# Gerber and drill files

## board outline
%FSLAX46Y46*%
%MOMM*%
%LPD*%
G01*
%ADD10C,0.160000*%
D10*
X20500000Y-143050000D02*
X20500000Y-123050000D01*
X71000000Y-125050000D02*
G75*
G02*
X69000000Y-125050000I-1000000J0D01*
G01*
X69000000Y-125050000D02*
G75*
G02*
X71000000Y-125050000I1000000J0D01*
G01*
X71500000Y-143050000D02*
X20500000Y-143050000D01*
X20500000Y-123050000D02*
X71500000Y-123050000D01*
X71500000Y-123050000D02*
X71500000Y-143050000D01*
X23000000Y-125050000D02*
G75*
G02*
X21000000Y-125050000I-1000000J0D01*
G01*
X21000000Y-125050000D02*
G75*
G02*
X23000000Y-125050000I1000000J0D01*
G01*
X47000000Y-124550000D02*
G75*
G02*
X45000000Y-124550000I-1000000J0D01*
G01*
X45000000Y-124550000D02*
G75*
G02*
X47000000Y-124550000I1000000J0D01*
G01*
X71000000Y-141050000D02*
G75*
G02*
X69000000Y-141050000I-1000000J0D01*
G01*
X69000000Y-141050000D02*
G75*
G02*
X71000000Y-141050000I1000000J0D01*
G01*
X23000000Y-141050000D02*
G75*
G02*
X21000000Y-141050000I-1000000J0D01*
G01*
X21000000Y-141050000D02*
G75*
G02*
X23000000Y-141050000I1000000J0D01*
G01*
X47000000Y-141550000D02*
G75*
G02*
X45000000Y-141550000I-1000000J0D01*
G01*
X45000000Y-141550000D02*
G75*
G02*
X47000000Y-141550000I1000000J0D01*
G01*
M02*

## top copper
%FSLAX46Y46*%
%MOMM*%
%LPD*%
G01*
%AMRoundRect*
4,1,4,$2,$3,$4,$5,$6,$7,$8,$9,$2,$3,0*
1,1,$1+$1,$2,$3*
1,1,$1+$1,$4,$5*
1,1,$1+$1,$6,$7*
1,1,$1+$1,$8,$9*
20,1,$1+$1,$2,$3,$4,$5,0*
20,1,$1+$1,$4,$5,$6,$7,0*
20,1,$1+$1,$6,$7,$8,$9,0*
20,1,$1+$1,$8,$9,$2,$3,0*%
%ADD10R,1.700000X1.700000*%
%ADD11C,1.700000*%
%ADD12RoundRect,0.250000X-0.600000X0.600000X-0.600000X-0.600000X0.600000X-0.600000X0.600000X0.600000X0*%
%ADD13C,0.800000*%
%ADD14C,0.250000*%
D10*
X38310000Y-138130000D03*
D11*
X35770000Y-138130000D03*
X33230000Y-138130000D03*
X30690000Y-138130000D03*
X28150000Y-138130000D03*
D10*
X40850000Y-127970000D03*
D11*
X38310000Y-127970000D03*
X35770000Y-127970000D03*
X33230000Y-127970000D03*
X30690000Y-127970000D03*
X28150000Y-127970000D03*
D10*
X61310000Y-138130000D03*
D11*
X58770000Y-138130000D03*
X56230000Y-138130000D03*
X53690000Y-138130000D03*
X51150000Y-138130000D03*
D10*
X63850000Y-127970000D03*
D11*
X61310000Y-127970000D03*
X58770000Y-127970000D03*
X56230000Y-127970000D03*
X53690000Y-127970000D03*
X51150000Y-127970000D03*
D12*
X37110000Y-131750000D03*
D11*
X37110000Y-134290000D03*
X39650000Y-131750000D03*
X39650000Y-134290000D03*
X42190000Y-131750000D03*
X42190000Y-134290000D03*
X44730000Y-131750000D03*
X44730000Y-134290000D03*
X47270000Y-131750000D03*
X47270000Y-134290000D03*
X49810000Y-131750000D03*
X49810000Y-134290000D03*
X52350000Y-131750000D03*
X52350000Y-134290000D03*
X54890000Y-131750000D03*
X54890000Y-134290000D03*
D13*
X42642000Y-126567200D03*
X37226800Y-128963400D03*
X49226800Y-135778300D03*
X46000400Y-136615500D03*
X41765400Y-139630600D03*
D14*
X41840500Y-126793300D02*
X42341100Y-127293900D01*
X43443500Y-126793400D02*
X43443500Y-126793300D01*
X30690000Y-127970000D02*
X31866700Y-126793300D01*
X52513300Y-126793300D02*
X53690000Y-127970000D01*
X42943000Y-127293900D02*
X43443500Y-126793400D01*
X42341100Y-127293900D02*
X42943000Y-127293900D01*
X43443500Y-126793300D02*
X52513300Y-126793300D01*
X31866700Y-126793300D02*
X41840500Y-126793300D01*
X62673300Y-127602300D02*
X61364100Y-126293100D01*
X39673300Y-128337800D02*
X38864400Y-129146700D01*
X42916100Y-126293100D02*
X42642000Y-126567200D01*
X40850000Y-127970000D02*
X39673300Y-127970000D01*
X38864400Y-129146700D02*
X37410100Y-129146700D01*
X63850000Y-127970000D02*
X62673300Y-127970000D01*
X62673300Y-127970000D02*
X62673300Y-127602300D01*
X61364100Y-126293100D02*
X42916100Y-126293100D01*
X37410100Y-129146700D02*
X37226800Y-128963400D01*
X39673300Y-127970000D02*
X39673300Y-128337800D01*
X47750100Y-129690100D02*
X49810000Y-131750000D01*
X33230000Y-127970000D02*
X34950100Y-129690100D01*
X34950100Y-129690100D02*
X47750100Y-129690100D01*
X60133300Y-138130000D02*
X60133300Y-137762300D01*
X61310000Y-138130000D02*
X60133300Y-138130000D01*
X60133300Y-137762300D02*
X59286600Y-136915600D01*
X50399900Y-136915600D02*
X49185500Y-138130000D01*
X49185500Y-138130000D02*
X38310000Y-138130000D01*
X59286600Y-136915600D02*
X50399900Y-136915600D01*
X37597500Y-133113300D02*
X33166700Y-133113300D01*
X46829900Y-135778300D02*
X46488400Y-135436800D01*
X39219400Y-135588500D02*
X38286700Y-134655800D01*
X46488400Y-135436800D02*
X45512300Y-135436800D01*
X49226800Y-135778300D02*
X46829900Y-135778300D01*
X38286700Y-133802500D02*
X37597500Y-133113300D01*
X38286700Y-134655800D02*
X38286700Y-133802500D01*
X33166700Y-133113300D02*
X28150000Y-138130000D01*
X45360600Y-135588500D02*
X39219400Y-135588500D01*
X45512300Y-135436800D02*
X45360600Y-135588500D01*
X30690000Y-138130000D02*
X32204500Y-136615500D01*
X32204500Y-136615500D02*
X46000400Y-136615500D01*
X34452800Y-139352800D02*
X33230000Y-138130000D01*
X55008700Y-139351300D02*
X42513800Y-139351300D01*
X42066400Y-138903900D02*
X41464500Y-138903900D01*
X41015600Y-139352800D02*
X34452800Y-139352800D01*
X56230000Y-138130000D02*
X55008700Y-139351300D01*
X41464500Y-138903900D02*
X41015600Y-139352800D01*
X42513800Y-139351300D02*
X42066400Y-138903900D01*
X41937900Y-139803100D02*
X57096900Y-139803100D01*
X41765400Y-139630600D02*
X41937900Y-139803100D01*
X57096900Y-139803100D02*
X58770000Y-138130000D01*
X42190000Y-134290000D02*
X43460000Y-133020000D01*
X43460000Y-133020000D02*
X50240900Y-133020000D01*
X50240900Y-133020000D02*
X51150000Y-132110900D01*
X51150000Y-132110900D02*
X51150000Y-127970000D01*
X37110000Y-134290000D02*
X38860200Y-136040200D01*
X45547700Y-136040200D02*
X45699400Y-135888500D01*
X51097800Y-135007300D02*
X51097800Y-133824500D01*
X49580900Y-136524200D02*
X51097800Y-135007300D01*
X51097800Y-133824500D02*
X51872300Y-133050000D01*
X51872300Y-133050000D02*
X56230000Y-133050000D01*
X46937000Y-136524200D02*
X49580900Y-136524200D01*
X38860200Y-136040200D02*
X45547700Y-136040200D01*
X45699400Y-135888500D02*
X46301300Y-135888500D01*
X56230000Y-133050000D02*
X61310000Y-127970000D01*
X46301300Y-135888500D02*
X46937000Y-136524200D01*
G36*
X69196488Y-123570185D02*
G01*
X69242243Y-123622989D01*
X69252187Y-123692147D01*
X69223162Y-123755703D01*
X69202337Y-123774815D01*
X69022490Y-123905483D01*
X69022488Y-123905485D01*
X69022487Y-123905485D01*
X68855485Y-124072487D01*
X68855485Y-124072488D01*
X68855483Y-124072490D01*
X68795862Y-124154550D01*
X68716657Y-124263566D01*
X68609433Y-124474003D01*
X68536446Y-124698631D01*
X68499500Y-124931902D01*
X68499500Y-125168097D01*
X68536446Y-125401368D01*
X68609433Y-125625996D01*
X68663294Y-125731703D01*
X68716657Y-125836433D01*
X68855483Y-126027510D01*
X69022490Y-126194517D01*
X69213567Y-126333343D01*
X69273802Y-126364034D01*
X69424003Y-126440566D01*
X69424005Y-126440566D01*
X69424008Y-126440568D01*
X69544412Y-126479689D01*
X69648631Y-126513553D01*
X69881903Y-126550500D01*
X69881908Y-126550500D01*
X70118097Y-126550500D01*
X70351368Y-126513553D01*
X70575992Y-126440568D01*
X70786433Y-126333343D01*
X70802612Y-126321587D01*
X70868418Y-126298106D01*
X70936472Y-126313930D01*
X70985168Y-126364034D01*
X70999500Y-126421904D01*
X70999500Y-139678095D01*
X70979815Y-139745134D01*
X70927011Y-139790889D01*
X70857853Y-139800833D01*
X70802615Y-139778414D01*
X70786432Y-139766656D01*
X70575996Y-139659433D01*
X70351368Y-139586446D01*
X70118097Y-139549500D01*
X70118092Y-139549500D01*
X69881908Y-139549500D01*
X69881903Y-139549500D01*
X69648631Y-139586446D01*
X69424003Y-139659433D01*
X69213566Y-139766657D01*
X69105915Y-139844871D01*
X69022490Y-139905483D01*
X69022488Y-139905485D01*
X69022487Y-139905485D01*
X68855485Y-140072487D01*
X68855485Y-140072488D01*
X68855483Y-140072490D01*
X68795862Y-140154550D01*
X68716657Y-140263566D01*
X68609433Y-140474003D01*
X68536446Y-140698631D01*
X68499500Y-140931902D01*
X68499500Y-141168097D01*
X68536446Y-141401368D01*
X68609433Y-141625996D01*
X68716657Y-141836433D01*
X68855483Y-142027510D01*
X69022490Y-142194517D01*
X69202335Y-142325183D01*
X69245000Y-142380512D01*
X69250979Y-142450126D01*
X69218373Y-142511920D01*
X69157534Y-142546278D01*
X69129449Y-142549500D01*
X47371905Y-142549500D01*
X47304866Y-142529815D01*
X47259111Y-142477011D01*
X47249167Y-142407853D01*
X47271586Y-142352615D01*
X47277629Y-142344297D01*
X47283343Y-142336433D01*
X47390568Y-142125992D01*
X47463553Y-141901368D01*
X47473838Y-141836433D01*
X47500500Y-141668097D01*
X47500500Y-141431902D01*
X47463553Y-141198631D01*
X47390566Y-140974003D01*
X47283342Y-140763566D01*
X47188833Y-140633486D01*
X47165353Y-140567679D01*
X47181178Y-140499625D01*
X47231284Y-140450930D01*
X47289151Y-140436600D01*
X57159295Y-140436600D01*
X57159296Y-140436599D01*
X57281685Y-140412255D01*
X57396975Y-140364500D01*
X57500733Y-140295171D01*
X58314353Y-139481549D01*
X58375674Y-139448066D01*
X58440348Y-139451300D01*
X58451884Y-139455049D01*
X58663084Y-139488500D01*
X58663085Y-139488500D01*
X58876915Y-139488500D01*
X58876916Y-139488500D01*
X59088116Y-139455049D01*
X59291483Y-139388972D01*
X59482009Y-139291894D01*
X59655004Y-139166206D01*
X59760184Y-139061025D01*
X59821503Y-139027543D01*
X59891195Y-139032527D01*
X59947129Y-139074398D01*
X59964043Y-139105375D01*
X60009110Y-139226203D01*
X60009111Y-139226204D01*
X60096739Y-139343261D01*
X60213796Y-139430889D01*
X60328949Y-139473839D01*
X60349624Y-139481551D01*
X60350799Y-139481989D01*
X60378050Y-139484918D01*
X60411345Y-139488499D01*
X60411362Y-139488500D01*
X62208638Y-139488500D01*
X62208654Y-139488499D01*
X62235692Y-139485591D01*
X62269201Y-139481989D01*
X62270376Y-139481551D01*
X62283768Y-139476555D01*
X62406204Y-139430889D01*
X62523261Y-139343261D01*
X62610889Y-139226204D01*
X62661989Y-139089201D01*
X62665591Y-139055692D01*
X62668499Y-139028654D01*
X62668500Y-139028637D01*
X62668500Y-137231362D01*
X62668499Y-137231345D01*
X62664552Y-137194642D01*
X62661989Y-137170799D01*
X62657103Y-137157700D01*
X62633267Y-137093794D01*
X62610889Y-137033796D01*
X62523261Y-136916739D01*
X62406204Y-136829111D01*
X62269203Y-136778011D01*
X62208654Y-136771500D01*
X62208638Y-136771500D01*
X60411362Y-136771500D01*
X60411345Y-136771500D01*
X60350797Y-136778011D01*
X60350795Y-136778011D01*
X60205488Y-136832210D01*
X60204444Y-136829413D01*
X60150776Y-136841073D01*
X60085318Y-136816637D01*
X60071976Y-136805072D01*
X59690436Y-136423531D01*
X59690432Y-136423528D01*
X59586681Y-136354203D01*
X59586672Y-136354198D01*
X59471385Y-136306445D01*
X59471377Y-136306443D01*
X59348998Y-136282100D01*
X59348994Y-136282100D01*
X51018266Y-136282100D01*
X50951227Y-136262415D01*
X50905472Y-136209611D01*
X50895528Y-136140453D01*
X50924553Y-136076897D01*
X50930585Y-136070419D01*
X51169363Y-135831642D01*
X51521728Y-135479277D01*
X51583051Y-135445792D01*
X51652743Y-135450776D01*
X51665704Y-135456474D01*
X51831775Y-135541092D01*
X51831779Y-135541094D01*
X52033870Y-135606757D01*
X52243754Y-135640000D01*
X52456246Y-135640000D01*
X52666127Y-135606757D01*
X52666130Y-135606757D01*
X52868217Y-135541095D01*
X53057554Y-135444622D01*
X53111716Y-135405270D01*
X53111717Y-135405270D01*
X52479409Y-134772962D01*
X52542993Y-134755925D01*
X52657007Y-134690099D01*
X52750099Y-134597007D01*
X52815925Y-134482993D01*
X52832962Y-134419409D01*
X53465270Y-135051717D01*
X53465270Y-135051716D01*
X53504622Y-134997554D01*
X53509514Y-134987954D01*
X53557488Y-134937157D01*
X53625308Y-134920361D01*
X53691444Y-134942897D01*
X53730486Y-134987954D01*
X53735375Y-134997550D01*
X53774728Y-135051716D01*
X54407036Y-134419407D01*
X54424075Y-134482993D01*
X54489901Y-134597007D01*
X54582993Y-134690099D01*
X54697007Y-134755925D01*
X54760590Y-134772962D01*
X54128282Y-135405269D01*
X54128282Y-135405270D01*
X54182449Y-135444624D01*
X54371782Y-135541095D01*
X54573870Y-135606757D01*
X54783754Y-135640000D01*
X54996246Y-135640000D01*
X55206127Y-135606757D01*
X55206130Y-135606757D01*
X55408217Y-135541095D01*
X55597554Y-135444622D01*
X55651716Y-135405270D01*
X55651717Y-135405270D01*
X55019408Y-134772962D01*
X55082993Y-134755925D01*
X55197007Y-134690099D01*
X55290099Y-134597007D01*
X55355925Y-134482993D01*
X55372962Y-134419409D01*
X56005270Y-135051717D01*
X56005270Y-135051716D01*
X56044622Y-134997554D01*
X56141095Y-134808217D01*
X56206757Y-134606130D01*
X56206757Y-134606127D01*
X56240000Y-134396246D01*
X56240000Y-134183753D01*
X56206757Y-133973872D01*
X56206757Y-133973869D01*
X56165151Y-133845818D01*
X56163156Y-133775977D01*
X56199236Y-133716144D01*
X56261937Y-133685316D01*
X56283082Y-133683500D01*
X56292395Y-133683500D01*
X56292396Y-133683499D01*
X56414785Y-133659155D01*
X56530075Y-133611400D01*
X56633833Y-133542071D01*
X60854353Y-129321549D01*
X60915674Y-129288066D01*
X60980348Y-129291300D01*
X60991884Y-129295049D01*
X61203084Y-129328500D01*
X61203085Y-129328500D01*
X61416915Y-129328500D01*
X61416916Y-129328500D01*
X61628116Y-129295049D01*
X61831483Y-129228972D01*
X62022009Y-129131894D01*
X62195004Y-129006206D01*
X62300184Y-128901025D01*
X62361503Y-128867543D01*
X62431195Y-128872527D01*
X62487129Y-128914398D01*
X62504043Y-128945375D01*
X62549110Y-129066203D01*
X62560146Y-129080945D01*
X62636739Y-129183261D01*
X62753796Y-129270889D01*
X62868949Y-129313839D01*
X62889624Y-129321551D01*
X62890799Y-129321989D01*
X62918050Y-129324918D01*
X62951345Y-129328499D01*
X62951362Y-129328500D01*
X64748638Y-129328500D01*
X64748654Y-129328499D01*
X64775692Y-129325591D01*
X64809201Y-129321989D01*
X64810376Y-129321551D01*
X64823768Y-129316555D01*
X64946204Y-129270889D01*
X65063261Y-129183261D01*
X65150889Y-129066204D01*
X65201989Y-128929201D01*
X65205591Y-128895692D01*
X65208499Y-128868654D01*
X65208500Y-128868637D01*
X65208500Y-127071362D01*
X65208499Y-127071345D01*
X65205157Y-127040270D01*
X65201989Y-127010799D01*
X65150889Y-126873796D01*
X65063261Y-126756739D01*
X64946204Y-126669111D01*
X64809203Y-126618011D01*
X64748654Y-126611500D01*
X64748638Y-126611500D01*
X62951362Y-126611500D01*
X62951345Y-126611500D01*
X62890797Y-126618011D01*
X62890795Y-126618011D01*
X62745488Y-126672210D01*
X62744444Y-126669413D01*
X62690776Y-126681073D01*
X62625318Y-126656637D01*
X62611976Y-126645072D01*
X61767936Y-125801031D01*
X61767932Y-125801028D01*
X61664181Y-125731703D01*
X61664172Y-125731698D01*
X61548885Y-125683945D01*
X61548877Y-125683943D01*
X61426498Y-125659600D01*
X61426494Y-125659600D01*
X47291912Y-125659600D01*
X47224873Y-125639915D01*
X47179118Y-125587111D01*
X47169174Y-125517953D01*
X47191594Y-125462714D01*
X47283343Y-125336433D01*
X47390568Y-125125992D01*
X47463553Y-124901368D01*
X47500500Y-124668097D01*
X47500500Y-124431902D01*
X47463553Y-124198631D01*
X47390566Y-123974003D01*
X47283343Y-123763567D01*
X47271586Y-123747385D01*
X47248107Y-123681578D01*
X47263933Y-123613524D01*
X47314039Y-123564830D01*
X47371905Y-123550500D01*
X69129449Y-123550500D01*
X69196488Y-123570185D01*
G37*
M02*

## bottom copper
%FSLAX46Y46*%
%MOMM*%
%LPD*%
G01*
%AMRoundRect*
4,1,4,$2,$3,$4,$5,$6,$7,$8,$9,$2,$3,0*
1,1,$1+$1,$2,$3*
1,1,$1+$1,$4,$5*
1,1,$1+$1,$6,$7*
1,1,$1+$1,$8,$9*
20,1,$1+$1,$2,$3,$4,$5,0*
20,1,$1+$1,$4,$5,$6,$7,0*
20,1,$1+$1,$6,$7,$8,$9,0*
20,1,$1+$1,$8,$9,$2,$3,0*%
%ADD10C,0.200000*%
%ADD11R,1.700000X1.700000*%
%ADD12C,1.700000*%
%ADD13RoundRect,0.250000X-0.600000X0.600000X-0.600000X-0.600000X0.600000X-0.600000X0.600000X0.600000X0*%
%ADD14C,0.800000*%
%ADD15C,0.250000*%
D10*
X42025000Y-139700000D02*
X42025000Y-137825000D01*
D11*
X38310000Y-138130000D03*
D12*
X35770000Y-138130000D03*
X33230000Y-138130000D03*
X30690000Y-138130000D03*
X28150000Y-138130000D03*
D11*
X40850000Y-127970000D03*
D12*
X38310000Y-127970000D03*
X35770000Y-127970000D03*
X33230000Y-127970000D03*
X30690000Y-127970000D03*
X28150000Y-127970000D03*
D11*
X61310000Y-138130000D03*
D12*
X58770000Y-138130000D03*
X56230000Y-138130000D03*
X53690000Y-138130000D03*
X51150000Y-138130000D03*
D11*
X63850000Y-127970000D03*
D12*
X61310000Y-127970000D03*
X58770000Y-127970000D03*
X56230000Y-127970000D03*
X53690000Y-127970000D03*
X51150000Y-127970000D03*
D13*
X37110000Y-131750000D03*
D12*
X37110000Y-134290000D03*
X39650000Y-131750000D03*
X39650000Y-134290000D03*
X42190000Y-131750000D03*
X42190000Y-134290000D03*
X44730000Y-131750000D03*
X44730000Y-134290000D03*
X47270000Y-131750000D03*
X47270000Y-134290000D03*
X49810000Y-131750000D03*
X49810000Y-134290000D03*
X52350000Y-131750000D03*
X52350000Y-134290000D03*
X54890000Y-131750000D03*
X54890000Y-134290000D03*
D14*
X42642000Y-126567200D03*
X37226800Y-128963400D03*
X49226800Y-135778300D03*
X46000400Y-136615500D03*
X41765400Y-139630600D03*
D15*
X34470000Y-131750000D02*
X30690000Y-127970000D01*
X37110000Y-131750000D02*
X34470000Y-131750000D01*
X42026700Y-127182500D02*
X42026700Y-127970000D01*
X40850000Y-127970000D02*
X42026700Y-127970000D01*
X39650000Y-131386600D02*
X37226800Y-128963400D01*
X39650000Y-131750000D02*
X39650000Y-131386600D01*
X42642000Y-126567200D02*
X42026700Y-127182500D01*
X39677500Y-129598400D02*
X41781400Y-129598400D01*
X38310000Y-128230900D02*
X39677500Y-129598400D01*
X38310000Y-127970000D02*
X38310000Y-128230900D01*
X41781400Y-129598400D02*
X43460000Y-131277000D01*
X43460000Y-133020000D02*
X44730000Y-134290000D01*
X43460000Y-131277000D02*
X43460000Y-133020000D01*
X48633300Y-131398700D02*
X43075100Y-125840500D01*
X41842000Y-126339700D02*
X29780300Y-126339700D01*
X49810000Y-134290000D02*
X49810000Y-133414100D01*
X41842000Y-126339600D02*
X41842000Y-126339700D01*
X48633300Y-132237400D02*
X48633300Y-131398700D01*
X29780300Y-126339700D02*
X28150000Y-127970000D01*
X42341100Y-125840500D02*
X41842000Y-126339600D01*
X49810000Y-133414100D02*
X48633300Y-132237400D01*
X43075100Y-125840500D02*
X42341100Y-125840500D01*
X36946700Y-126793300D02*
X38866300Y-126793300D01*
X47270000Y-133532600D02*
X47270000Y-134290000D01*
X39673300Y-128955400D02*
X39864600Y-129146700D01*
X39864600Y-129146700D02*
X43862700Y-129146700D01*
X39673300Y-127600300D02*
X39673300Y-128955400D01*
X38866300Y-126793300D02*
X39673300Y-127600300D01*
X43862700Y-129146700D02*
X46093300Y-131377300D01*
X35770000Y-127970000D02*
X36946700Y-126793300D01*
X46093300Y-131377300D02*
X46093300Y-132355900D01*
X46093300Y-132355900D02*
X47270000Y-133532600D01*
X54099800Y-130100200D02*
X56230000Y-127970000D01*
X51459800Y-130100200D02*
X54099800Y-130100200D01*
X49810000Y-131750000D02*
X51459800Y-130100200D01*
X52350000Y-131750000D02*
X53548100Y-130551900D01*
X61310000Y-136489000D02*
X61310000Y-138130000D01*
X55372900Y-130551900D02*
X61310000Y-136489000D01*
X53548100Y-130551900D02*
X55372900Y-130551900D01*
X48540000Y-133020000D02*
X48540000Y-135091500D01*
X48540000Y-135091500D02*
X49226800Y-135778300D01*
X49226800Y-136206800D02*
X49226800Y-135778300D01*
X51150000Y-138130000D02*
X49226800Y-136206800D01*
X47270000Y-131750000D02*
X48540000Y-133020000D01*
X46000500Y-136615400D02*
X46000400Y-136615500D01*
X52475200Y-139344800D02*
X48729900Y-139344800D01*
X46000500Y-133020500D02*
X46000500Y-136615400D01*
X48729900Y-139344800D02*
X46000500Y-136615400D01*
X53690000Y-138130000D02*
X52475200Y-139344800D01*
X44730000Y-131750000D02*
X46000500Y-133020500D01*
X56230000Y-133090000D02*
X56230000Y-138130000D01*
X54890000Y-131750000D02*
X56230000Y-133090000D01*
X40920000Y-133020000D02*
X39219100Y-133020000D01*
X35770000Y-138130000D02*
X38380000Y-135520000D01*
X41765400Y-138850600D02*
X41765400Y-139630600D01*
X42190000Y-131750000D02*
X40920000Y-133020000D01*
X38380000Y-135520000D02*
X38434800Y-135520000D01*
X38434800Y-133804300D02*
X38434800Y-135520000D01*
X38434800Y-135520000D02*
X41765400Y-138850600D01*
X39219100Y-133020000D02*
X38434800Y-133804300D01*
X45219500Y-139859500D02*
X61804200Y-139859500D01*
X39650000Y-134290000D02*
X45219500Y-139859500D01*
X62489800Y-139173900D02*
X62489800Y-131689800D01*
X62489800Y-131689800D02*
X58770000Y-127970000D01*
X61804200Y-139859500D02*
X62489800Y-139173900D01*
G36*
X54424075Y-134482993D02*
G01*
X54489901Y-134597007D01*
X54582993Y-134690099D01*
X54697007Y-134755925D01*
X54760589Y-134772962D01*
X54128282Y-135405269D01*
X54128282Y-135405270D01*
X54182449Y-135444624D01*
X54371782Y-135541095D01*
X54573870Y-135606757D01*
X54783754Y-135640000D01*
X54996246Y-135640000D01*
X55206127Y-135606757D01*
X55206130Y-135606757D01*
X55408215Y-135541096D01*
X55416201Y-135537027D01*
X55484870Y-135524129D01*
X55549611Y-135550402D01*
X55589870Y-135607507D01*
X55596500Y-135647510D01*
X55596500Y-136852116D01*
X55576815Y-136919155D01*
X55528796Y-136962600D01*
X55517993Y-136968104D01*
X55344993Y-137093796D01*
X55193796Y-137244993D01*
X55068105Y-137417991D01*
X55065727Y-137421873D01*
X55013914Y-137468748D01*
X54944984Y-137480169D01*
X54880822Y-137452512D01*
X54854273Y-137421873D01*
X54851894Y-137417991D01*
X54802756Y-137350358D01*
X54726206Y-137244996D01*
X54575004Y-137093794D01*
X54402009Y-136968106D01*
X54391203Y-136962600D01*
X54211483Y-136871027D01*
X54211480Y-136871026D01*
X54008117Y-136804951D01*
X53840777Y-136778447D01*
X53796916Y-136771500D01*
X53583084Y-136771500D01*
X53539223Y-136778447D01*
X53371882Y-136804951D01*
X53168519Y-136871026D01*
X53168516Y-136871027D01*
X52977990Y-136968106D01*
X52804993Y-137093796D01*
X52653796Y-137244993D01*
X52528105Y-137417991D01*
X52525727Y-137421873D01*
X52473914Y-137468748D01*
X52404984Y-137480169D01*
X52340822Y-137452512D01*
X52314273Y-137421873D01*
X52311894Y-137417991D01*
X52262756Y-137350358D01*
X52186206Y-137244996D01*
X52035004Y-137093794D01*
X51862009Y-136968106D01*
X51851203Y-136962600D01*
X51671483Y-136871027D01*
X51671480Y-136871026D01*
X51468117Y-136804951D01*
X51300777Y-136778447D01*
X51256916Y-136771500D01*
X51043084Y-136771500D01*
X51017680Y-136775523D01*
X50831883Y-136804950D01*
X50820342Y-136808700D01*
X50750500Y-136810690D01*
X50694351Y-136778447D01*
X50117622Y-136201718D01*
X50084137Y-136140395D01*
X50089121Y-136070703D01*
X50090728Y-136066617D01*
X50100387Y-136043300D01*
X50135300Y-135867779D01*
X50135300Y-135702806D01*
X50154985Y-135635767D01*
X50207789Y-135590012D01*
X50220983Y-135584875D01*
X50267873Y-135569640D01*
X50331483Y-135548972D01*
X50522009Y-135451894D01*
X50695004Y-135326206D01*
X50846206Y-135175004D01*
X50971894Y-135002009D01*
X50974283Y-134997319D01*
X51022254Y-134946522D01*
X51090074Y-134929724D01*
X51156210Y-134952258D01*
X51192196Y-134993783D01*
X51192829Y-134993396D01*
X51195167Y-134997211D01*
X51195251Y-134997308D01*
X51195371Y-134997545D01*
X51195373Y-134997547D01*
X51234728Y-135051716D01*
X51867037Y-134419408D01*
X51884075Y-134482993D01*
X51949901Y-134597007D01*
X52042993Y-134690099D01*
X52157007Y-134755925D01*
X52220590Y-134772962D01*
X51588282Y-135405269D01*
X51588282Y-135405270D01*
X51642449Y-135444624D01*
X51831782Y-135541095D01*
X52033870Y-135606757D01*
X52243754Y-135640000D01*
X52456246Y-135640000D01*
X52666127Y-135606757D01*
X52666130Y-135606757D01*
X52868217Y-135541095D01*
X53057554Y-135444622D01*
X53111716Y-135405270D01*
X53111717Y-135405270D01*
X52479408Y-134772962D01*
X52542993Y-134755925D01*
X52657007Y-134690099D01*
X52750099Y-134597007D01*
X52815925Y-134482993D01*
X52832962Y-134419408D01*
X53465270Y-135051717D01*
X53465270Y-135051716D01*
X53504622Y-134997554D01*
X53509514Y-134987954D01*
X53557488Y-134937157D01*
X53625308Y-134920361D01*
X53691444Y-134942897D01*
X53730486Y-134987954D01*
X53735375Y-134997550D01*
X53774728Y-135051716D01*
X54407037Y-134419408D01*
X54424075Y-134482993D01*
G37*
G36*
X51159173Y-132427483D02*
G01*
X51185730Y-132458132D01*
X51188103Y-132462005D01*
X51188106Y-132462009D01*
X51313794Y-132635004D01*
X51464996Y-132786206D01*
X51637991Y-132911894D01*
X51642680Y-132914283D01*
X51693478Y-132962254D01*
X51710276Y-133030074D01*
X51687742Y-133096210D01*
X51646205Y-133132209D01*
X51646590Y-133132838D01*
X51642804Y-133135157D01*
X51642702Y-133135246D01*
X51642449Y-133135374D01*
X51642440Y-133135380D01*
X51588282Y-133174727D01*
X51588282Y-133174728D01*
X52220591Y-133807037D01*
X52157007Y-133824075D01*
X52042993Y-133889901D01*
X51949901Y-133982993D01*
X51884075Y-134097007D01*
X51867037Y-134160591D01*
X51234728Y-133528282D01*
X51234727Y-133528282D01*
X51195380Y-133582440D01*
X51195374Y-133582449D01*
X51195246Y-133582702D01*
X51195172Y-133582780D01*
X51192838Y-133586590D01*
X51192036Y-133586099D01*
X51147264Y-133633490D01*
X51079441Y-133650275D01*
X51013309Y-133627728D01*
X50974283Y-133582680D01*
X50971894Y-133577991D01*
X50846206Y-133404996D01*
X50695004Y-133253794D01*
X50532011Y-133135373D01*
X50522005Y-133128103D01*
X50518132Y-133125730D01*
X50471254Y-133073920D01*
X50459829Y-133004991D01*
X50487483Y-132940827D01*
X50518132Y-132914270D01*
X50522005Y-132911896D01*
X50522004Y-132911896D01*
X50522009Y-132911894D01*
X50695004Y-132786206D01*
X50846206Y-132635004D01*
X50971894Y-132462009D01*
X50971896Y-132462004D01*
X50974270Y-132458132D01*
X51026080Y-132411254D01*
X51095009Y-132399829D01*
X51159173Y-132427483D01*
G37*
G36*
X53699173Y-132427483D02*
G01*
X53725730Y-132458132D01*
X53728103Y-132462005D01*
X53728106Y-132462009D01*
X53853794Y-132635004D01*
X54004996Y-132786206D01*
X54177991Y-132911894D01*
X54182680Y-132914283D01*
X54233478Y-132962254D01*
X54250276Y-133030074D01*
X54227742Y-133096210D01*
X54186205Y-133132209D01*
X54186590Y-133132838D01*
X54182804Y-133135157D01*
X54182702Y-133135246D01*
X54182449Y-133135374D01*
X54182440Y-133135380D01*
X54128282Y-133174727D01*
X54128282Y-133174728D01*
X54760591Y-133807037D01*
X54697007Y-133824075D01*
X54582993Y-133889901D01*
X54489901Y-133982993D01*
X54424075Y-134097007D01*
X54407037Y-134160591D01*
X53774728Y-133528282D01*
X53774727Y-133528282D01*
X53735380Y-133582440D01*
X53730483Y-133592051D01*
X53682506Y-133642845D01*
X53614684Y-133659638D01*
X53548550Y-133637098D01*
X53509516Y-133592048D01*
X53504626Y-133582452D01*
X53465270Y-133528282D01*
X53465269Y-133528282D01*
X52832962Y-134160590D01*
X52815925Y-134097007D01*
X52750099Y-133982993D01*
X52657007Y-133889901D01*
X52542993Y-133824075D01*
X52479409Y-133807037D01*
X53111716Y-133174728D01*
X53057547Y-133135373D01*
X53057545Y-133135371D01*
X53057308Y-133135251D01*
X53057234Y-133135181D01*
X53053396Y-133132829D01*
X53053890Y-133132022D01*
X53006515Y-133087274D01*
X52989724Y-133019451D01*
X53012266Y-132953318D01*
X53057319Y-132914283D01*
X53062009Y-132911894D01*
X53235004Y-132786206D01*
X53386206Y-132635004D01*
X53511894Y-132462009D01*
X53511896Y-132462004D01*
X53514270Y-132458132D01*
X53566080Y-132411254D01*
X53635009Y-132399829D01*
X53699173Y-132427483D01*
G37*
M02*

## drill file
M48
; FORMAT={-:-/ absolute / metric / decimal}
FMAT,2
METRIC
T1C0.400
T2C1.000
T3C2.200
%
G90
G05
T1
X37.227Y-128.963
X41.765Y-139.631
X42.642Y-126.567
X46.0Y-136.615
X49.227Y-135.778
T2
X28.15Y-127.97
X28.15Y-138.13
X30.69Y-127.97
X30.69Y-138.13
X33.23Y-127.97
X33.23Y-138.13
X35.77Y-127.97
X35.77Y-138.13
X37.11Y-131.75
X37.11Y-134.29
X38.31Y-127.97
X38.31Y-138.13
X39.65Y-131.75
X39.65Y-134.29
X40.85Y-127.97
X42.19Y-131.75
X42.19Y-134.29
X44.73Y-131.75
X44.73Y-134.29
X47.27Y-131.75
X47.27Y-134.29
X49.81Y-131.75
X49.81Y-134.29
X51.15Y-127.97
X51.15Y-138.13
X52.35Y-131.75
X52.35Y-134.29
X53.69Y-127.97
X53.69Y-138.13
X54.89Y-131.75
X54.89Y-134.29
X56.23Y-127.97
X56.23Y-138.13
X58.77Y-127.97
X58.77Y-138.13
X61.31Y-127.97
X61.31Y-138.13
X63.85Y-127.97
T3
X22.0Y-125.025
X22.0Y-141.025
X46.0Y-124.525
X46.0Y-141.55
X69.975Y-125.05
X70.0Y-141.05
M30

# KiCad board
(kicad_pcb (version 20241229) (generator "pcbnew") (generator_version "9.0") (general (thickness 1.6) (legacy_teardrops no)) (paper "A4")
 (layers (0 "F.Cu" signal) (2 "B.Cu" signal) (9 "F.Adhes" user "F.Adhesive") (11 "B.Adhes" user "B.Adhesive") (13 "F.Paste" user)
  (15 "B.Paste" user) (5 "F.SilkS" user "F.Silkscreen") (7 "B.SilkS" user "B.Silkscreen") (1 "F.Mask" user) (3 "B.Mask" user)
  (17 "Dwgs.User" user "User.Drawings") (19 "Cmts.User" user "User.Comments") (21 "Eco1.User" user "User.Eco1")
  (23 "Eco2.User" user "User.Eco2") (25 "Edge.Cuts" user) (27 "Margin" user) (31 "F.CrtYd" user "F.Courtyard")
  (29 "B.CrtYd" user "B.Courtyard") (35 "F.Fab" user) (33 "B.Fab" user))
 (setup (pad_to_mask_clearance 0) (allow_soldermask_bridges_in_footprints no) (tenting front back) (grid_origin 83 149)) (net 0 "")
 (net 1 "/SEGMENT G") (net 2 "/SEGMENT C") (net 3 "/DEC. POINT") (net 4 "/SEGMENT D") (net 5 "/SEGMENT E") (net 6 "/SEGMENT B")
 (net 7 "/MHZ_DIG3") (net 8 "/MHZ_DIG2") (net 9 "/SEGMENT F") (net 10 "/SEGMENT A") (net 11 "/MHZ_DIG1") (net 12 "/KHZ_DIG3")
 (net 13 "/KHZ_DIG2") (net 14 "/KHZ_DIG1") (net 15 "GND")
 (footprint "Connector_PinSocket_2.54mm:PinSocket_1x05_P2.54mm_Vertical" (layer "F.Cu") (at 38.31 138.13 -90)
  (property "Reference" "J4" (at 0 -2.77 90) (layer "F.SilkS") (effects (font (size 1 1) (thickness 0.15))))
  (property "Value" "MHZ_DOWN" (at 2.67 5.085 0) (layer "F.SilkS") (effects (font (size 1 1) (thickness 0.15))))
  (pad "1" thru_hole rect (at 0 0 270) (size 1.7 1.7) (drill 1) (layers "*.Cu" "*.Mask") (remove_unused_layers no) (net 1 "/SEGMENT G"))
  (pad "2" thru_hole circle (at 0 2.54 270) (size 1.7 1.7) (drill 1) (layers "*.Cu" "*.Mask") (remove_unused_layers no) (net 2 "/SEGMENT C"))
  (pad "3" thru_hole circle (at 0 5.08 270) (size 1.7 1.7) (drill 1) (layers "*.Cu" "*.Mask") (remove_unused_layers no)
   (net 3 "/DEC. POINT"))
  (pad "4" thru_hole circle (at 0 7.62 270) (size 1.7 1.7) (drill 1) (layers "*.Cu" "*.Mask") (remove_unused_layers no) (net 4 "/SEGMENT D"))
  (pad "5" thru_hole circle (at 0 10.16 270) (size 1.7 1.7) (drill 1) (layers "*.Cu" "*.Mask") (remove_unused_layers no)
   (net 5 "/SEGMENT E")))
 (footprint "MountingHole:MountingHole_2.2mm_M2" (layer "F.Cu") (at 69.975 125.05)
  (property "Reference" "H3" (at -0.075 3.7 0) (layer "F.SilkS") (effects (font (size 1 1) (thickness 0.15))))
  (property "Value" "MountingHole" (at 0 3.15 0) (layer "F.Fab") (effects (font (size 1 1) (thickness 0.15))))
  (pad "" np_thru_hole circle (at 0 0) (size 2.2 2.2) (drill 2.2) (layers "*.Cu" "*.Mask")))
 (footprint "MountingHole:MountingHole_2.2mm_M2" (layer "F.Cu") (at 70 141.05)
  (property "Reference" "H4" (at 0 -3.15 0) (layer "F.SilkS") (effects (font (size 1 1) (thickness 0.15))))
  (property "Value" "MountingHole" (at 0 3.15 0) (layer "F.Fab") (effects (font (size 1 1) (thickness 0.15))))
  (pad "" np_thru_hole circle (at 0 0) (size 2.2 2.2) (drill 2.2) (layers "*.Cu" "*.Mask")))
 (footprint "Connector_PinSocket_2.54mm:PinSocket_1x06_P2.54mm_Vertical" (layer "F.Cu") (at 40.85 127.97 -90)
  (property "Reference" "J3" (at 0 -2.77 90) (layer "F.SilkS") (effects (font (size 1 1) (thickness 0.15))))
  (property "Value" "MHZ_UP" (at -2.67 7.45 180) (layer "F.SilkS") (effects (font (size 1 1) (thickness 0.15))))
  (pad "1" thru_hole rect (at 0 0 270) (size 1.7 1.7) (drill 1) (layers "*.Cu" "*.Mask") (remove_unused_layers no) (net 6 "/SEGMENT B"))
  (pad "2" thru_hole circle (at 0 2.54 270) (size 1.7 1.7) (drill 1) (layers "*.Cu" "*.Mask") (remove_unused_layers no) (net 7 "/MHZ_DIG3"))
  (pad "3" thru_hole circle (at 0 5.08 270) (size 1.7 1.7) (drill 1) (layers "*.Cu" "*.Mask") (remove_unused_layers no) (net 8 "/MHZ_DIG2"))
  (pad "4" thru_hole circle (at 0 7.62 270) (size 1.7 1.7) (drill 1) (layers "*.Cu" "*.Mask") (remove_unused_layers no) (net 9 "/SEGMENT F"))
  (pad "5" thru_hole circle (at 0 10.16 270) (size 1.7 1.7) (drill 1) (layers "*.Cu" "*.Mask") (remove_unused_layers no)
   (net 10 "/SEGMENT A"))
  (pad "6" thru_hole circle (at 0 12.7 270) (size 1.7 1.7) (drill 1) (layers "*.Cu" "*.Mask") (remove_unused_layers no) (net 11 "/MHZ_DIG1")))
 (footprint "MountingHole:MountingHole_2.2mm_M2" (layer "F.Cu") (at 46 141.55 180)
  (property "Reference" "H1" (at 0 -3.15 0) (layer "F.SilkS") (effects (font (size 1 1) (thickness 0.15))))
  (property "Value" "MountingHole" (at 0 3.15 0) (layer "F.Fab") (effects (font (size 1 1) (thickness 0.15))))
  (pad "" np_thru_hole circle (at 0 0 180) (size 2.2 2.2) (drill 2.2) (layers "*.Cu" "*.Mask")))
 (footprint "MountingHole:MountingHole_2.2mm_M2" (layer "F.Cu") (at 22 125.025)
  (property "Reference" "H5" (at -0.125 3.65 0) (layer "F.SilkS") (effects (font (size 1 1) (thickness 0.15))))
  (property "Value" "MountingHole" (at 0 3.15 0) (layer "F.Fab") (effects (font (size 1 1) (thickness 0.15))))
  (pad "" np_thru_hole circle (at 0 0) (size 2.2 2.2) (drill 2.2) (layers "*.Cu" "*.Mask")))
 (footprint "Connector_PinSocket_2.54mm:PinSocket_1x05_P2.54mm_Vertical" (layer "F.Cu") (at 61.31 138.13 -90)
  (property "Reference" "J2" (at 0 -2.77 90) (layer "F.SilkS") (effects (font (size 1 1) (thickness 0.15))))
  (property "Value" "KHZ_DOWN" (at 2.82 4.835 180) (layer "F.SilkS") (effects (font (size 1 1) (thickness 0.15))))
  (pad "1" thru_hole rect (at 0 0 270) (size 1.7 1.7) (drill 1) (layers "*.Cu" "*.Mask") (remove_unused_layers no) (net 1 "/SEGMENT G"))
  (pad "2" thru_hole circle (at 0 2.54 270) (size 1.7 1.7) (drill 1) (layers "*.Cu" "*.Mask") (remove_unused_layers no) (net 2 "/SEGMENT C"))
  (pad "3" thru_hole circle (at 0 5.08 270) (size 1.7 1.7) (drill 1) (layers "*.Cu" "*.Mask") (remove_unused_layers no)
   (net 3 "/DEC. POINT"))
  (pad "4" thru_hole circle (at 0 7.62 270) (size 1.7 1.7) (drill 1) (layers "*.Cu" "*.Mask") (remove_unused_layers no) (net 4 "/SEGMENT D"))
  (pad "5" thru_hole circle (at 0 10.16 270) (size 1.7 1.7) (drill 1) (layers "*.Cu" "*.Mask") (remove_unused_layers no)
   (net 5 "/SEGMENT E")))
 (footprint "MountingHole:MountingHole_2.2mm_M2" (layer "F.Cu") (at 46 124.525 180)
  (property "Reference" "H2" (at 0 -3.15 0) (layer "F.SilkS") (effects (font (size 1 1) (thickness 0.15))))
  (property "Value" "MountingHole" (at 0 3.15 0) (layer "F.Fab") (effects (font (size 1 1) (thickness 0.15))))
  (pad "" np_thru_hole circle (at 0 0 180) (size 2.2 2.2) (drill 2.2) (layers "*.Cu" "*.Mask")))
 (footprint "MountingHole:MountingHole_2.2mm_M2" (layer "F.Cu") (at 22 141.025)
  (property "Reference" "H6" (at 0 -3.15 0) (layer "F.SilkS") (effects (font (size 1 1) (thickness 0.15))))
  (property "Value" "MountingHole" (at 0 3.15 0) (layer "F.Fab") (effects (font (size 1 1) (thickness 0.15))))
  (pad "" np_thru_hole circle (at 0 0) (size 2.2 2.2) (drill 2.2) (layers "*.Cu" "*.Mask")))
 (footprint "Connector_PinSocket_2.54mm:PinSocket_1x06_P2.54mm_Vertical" (layer "F.Cu") (at 63.85 127.97 -90)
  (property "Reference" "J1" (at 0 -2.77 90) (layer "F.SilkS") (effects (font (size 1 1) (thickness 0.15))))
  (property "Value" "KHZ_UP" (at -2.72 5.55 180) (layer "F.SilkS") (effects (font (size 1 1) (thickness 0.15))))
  (pad "1" thru_hole rect (at 0 0 270) (size 1.7 1.7) (drill 1) (layers "*.Cu" "*.Mask") (remove_unused_layers no) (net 6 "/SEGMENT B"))
  (pad "2" thru_hole circle (at 0 2.54 270) (size 1.7 1.7) (drill 1) (layers "*.Cu" "*.Mask") (remove_unused_layers no) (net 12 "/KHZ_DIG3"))
  (pad "3" thru_hole circle (at 0 5.08 270) (size 1.7 1.7) (drill 1) (layers "*.Cu" "*.Mask") (remove_unused_layers no) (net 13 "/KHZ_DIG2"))
  (pad "4" thru_hole circle (at 0 7.62 270) (size 1.7 1.7) (drill 1) (layers "*.Cu" "*.Mask") (remove_unused_layers no) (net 9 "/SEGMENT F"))
  (pad "5" thru_hole circle (at 0 10.16 270) (size 1.7 1.7) (drill 1) (layers "*.Cu" "*.Mask") (remove_unused_layers no)
   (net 10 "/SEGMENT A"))
  (pad "6" thru_hole circle (at 0 12.7 270) (size 1.7 1.7) (drill 1) (layers "*.Cu" "*.Mask") (remove_unused_layers no) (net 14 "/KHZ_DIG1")))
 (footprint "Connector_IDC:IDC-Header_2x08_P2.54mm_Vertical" (layer "B.Cu") (at 37.11 131.75 -90)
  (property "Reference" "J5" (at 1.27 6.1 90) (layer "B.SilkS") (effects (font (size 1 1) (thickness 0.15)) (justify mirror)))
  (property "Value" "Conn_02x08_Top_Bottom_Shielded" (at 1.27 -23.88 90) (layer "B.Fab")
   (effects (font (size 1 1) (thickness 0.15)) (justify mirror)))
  (pad "1" thru_hole roundrect (at 0 0 270) (size 1.7 1.7) (drill 1) (layers "*.Cu" "*.Mask") (remove_unused_layers no)
   (roundrect_rratio 0.147059) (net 10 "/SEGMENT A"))
  (pad "2" thru_hole circle (at 2.54 0 270) (size 1.7 1.7) (drill 1) (layers "*.Cu" "*.Mask") (remove_unused_layers no) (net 12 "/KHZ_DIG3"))
  (pad "3" thru_hole circle (at 0 -2.54 270) (size 1.7 1.7) (drill 1) (layers "*.Cu" "*.Mask") (remove_unused_layers no)
   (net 6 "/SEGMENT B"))
  (pad "4" thru_hole circle (at 2.54 -2.54 270) (size 1.7 1.7) (drill 1) (layers "*.Cu" "*.Mask") (remove_unused_layers no)
   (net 13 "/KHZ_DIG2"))
  (pad "5" thru_hole circle (at 0 -5.08 270) (size 1.7 1.7) (drill 1) (layers "*.Cu" "*.Mask") (remove_unused_layers no)
   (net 2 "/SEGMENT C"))
  (pad "6" thru_hole circle (at 2.54 -5.08 270) (size 1.7 1.7) (drill 1) (layers "*.Cu" "*.Mask") (remove_unused_layers no)
   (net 14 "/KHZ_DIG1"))
  (pad "7" thru_hole circle (at 0 -7.62 270) (size 1.7 1.7) (drill 1) (layers "*.Cu" "*.Mask") (remove_unused_layers no)
   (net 4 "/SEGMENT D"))
  (pad "8" thru_hole circle (at 2.54 -7.62 270) (size 1.7 1.7) (drill 1) (layers "*.Cu" "*.Mask") (remove_unused_layers no)
   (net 7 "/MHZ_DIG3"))
  (pad "9" thru_hole circle (at 0 -10.16 270) (size 1.7 1.7) (drill 1) (layers "*.Cu" "*.Mask") (remove_unused_layers no)
   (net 5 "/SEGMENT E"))
  (pad "10" thru_hole circle (at 2.54 -10.16 270) (size 1.7 1.7) (drill 1) (layers "*.Cu" "*.Mask") (remove_unused_layers no)
   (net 8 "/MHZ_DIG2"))
  (pad "11" thru_hole circle (at 0 -12.7 270) (size 1.7 1.7) (drill 1) (layers "*.Cu" "*.Mask") (remove_unused_layers no)
   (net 9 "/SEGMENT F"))
  (pad "12" thru_hole circle (at 2.54 -12.7 270) (size 1.7 1.7) (drill 1) (layers "*.Cu" "*.Mask") (remove_unused_layers no)
   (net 11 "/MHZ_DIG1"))
  (pad "13" thru_hole circle (at 0 -15.24 270) (size 1.7 1.7) (drill 1) (layers "*.Cu" "*.Mask") (remove_unused_layers no)
   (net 1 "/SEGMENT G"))
  (pad "14" thru_hole circle (at 2.54 -15.24 270) (size 1.7 1.7) (drill 1) (layers "*.Cu" "*.Mask") (remove_unused_layers no) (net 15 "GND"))
  (pad "15" thru_hole circle (at 0 -17.78 270) (size 1.7 1.7) (drill 1) (layers "*.Cu" "*.Mask") (remove_unused_layers no)
   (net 3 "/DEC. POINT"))
  (pad "16" thru_hole circle (at 2.54 -17.78 270) (size 1.7 1.7) (drill 1) (layers "*.Cu" "*.Mask") (remove_unused_layers no) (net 15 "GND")))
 (gr_line (start 42.025 139.7) (end 42.025 137.825) (stroke (width 0.2) (type default)) (layer "B.Cu") (net 2))
 (gr_line (start 20.5 143.05) (end 20.5 123.05) (stroke (width 0.16) (type solid)) (layer "Edge.Cuts"))
 (gr_circle (center 70 125.05) (end 71 125.05) (stroke (width 0.16) (type solid)) (fill no) (layer "Edge.Cuts"))
 (gr_line (start 71.5 143.05) (end 20.5 143.05) (stroke (width 0.16) (type solid)) (layer "Edge.Cuts"))
 (gr_line (start 20.5 123.05) (end 71.5 123.05) (stroke (width 0.16) (type solid)) (layer "Edge.Cuts"))
 (gr_line (start 71.5 123.05) (end 71.5 143.05) (stroke (width 0.16) (type solid)) (layer "Edge.Cuts"))
 (gr_circle (center 22 125.05) (end 23 125.05) (stroke (width 0.16) (type solid)) (fill no) (layer "Edge.Cuts"))
 (gr_circle (center 46 124.55) (end 47 124.55) (stroke (width 0.16) (type solid)) (fill no) (layer "Edge.Cuts"))
 (gr_circle (center 70 141.05) (end 71 141.05) (stroke (width 0.16) (type solid)) (fill no) (layer "Edge.Cuts"))
 (gr_circle (center 22 141.05) (end 23 141.05) (stroke (width 0.16) (type solid)) (fill no) (layer "Edge.Cuts"))
 (gr_circle (center 46 141.55) (end 47 141.55) (stroke (width 0.16) (type solid)) (fill no) (layer "Edge.Cuts"))
 (segment (start 41.8405 126.7933) (end 42.3411 127.2939) (width 0.25) (layer "F.Cu") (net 10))
 (segment (start 43.4435 126.7934) (end 43.4435 126.7933) (width 0.25) (layer "F.Cu") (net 10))
 (segment (start 30.69 127.97) (end 31.8667 126.7933) (width 0.25) (layer "F.Cu") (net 10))
 (segment (start 52.5133 126.7933) (end 53.69 127.97) (width 0.25) (layer "F.Cu") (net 10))
 (segment (start 42.943 127.2939) (end 43.4435 126.7934) (width 0.25) (layer "F.Cu") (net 10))
 (segment (start 42.3411 127.2939) (end 42.943 127.2939) (width 0.25) (layer "F.Cu") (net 10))
 (segment (start 43.4435 126.7933) (end 52.5133 126.7933) (width 0.25) (layer "F.Cu") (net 10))
 (segment (start 31.8667 126.7933) (end 41.8405 126.7933) (width 0.25) (layer "F.Cu") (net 10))
 (segment (start 34.47 131.75) (end 30.69 127.97) (width 0.25) (layer "B.Cu") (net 10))
 (segment (start 37.11 131.75) (end 34.47 131.75) (width 0.25) (layer "B.Cu") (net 10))
 (segment (start 62.6733 127.6023) (end 61.3641 126.2931) (width 0.25) (layer "F.Cu") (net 6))
 (segment (start 39.6733 128.3378) (end 38.8644 129.1467) (width 0.25) (layer "F.Cu") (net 6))
 (segment (start 42.9161 126.2931) (end 42.642 126.5672) (width 0.25) (layer "F.Cu") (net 6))
 (segment (start 40.85 127.97) (end 39.6733 127.97) (width 0.25) (layer "F.Cu") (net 6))
 (segment (start 38.8644 129.1467) (end 37.4101 129.1467) (width 0.25) (layer "F.Cu") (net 6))
 (segment (start 63.85 127.97) (end 62.6733 127.97) (width 0.25) (layer "F.Cu") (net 6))
 (segment (start 62.6733 127.97) (end 62.6733 127.6023) (width 0.25) (layer "F.Cu") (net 6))
 (segment (start 61.3641 126.2931) (end 42.9161 126.2931) (width 0.25) (layer "F.Cu") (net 6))
 (segment (start 37.4101 129.1467) (end 37.2268 128.9634) (width 0.25) (layer "F.Cu") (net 6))
 (segment (start 39.6733 127.97) (end 39.6733 128.3378) (width 0.25) (layer "F.Cu") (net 6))
 (via (at 42.642 126.5672) (size 0.8) (drill 0.4) (layers "F.Cu" "B.Cu") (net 6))
 (via (at 37.2268 128.9634) (size 0.8) (drill 0.4) (layers "F.Cu" "B.Cu") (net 6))
 (segment (start 42.0267 127.1825) (end 42.0267 127.97) (width 0.25) (layer "B.Cu") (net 6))
 (segment (start 40.85 127.97) (end 42.0267 127.97) (width 0.25) (layer "B.Cu") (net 6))
 (segment (start 39.65 131.3866) (end 37.2268 128.9634) (width 0.25) (layer "B.Cu") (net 6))
 (segment (start 39.65 131.75) (end 39.65 131.3866) (width 0.25) (layer "B.Cu") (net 6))
 (segment (start 42.642 126.5672) (end 42.0267 127.1825) (width 0.25) (layer "B.Cu") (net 6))
 (segment (start 39.6775 129.5984) (end 41.7814 129.5984) (width 0.25) (layer "B.Cu") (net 7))
 (segment (start 38.31 128.2309) (end 39.6775 129.5984) (width 0.25) (layer "B.Cu") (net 7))
 (segment (start 38.31 127.97) (end 38.31 128.2309) (width 0.25) (layer "B.Cu") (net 7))
 (segment (start 41.7814 129.5984) (end 43.46 131.277) (width 0.25) (layer "B.Cu") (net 7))
 (segment (start 43.46 133.02) (end 44.73 134.29) (width 0.25) (layer "B.Cu") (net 7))
 (segment (start 43.46 131.277) (end 43.46 133.02) (width 0.25) (layer "B.Cu") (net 7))
 (segment (start 48.6333 131.3987) (end 43.0751 125.8405) (width 0.25) (layer "B.Cu") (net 11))
 (segment (start 41.842 126.3397) (end 29.7803 126.3397) (width 0.25) (layer "B.Cu") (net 11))
 (segment (start 49.81 134.29) (end 49.81 133.4141) (width 0.25) (layer "B.Cu") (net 11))
 (segment (start 41.842 126.3396) (end 41.842 126.3397) (width 0.25) (layer "B.Cu") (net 11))
 (segment (start 48.6333 132.2374) (end 48.6333 131.3987) (width 0.25) (layer "B.Cu") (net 11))
 (segment (start 29.7803 126.3397) (end 28.15 127.97) (width 0.25) (layer "B.Cu") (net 11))
 (segment (start 42.3411 125.8405) (end 41.842 126.3396) (width 0.25) (layer "B.Cu") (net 11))
 (segment (start 49.81 133.4141) (end 48.6333 132.2374) (width 0.25) (layer "B.Cu") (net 11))
 (segment (start 43.0751 125.8405) (end 42.3411 125.8405) (width 0.25) (layer "B.Cu") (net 11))
 (segment (start 36.9467 126.7933) (end 38.8663 126.7933) (width 0.25) (layer "B.Cu") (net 8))
 (segment (start 47.27 133.5326) (end 47.27 134.29) (width 0.25) (layer "B.Cu") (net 8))
 (segment (start 39.6733 128.9554) (end 39.8646 129.1467) (width 0.25) (layer "B.Cu") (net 8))
 (segment (start 39.8646 129.1467) (end 43.8627 129.1467) (width 0.25) (layer "B.Cu") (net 8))
 (segment (start 39.6733 127.6003) (end 39.6733 128.9554) (width 0.25) (layer "B.Cu") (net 8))
 (segment (start 38.8663 126.7933) (end 39.6733 127.6003) (width 0.25) (layer "B.Cu") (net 8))
 (segment (start 43.8627 129.1467) (end 46.0933 131.3773) (width 0.25) (layer "B.Cu") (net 8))
 (segment (start 35.77 127.97) (end 36.9467 126.7933) (width 0.25) (layer "B.Cu") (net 8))
 (segment (start 46.0933 131.3773) (end 46.0933 132.3559) (width 0.25) (layer "B.Cu") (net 8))
 (segment (start 46.0933 132.3559) (end 47.27 133.5326) (width 0.25) (layer "B.Cu") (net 8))
 (segment (start 47.7501 129.6901) (end 49.81 131.75) (width 0.25) (layer "F.Cu") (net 9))
 (segment (start 33.23 127.97) (end 34.9501 129.6901) (width 0.25) (layer "F.Cu") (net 9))
 (segment (start 34.9501 129.6901) (end 47.7501 129.6901) (width 0.25) (layer "F.Cu") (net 9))
 (segment (start 54.0998 130.1002) (end 56.23 127.97) (width 0.25) (layer "B.Cu") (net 9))
 (segment (start 51.4598 130.1002) (end 54.0998 130.1002) (width 0.25) (layer "B.Cu") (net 9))
 (segment (start 49.81 131.75) (end 51.4598 130.1002) (width 0.25) (layer "B.Cu") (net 9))
 (segment (start 60.1333 138.13) (end 60.1333 137.7623) (width 0.25) (layer "F.Cu") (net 1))
 (segment (start 61.31 138.13) (end 60.1333 138.13) (width 0.25) (layer "F.Cu") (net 1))
 (segment (start 60.1333 137.7623) (end 59.2866 136.9156) (width 0.25) (layer "F.Cu") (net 1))
 (segment (start 50.3999 136.9156) (end 49.1855 138.13) (width 0.25) (layer "F.Cu") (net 1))
 (segment (start 49.1855 138.13) (end 38.31 138.13) (width 0.25) (layer "F.Cu") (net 1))
 (segment (start 59.2866 136.9156) (end 50.3999 136.9156) (width 0.25) (layer "F.Cu") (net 1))
 (segment (start 52.35 131.75) (end 53.5481 130.5519) (width 0.25) (layer "B.Cu") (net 1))
 (segment (start 61.31 136.489) (end 61.31 138.13) (width 0.25) (layer "B.Cu") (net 1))
 (segment (start 55.3729 130.5519) (end 61.31 136.489) (width 0.25) (layer "B.Cu") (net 1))
 (segment (start 53.5481 130.5519) (end 55.3729 130.5519) (width 0.25) (layer "B.Cu") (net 1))
 (segment (start 37.5975 133.1133) (end 33.1667 133.1133) (width 0.25) (layer "F.Cu") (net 5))
 (segment (start 46.8299 135.7783) (end 46.4884 135.4368) (width 0.25) (layer "F.Cu") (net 5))
 (segment (start 39.2194 135.5885) (end 38.2867 134.6558) (width 0.25) (layer "F.Cu") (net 5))
 (segment (start 46.4884 135.4368) (end 45.5123 135.4368) (width 0.25) (layer "F.Cu") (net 5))
 (segment (start 49.2268 135.7783) (end 46.8299 135.7783) (width 0.25) (layer "F.Cu") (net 5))
 (segment (start 38.2867 133.8025) (end 37.5975 133.1133) (width 0.25) (layer "F.Cu") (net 5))
 (segment (start 38.2867 134.6558) (end 38.2867 133.8025) (width 0.25) (layer "F.Cu") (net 5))
 (segment (start 33.1667 133.1133) (end 28.15 138.13) (width 0.25) (layer "F.Cu") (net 5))
 (segment (start 45.3606 135.5885) (end 39.2194 135.5885) (width 0.25) (layer "F.Cu") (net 5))
 (segment (start 45.5123 135.4368) (end 45.3606 135.5885) (width 0.25) (layer "F.Cu") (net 5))
 (via (at 49.2268 135.7783) (size 0.8) (drill 0.4) (layers "F.Cu" "B.Cu") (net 5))
 (segment (start 48.54 133.02) (end 48.54 135.0915) (width 0.25) (layer "B.Cu") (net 5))
 (segment (start 48.54 135.0915) (end 49.2268 135.7783) (width 0.25) (layer "B.Cu") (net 5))
 (segment (start 49.2268 136.2068) (end 49.2268 135.7783) (width 0.25) (layer "B.Cu") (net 5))
 (segment (start 51.15 138.13) (end 49.2268 136.2068) (width 0.25) (layer "B.Cu") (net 5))
 (segment (start 47.27 131.75) (end 48.54 133.02) (width 0.25) (layer "B.Cu") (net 5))
 (segment (start 30.69 138.13) (end 32.2045 136.6155) (width 0.25) (layer "F.Cu") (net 4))
 (segment (start 32.2045 136.6155) (end 46.0004 136.6155) (width 0.25) (layer "F.Cu") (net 4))
 (via (at 46.0004 136.6155) (size 0.8) (drill 0.4) (layers "F.Cu" "B.Cu") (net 4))
 (segment (start 46.0005 136.6154) (end 46.0004 136.6155) (width 0.25) (layer "B.Cu") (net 4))
 (segment (start 52.4752 139.3448) (end 48.7299 139.3448) (width 0.25) (layer "B.Cu") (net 4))
 (segment (start 46.0005 133.0205) (end 46.0005 136.6154) (width 0.25) (layer "B.Cu") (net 4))
 (segment (start 48.7299 139.3448) (end 46.0005 136.6154) (width 0.25) (layer "B.Cu") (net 4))
 (segment (start 53.69 138.13) (end 52.4752 139.3448) (width 0.25) (layer "B.Cu") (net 4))
 (segment (start 44.73 131.75) (end 46.0005 133.0205) (width 0.25) (layer "B.Cu") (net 4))
 (segment (start 34.4528 139.3528) (end 33.23 138.13) (width 0.25) (layer "F.Cu") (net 3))
 (segment (start 55.0087 139.3513) (end 42.5138 139.3513) (width 0.25) (layer "F.Cu") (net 3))
 (segment (start 42.0664 138.9039) (end 41.4645 138.9039) (width 0.25) (layer "F.Cu") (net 3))
 (segment (start 41.0156 139.3528) (end 34.4528 139.3528) (width 0.25) (layer "F.Cu") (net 3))
 (segment (start 56.23 138.13) (end 55.0087 139.3513) (width 0.25) (layer "F.Cu") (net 3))
 (segment (start 41.4645 138.9039) (end 41.0156 139.3528) (width 0.25) (layer "F.Cu") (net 3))
 (segment (start 42.5138 139.3513) (end 42.0664 138.9039) (width 0.25) (layer "F.Cu") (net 3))
 (segment (start 56.23 133.09) (end 56.23 138.13) (width 0.25) (layer "B.Cu") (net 3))
 (segment (start 54.89 131.75) (end 56.23 133.09) (width 0.25) (layer "B.Cu") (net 3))
 (segment (start 41.9379 139.8031) (end 57.0969 139.8031) (width 0.25) (layer "F.Cu") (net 2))
 (segment (start 41.7654 139.6306) (end 41.9379 139.8031) (width 0.25) (layer "F.Cu") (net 2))
 (segment (start 57.0969 139.8031) (end 58.77 138.13) (width 0.25) (layer "F.Cu") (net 2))
 (via (at 41.7654 139.6306) (size 0.8) (drill 0.4) (layers "F.Cu" "B.Cu") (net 2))
 (segment (start 40.92 133.02) (end 39.2191 133.02) (width 0.25) (layer "B.Cu") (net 2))
 (segment (start 35.77 138.13) (end 38.38 135.52) (width 0.25) (layer "B.Cu") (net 2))
 (segment (start 41.7654 138.8506) (end 41.7654 139.6306) (width 0.25) (layer "B.Cu") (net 2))
 (segment (start 42.19 131.75) (end 40.92 133.02) (width 0.25) (layer "B.Cu") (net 2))
 (segment (start 38.38 135.52) (end 38.4348 135.52) (width 0.25) (layer "B.Cu") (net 2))
 (segment (start 38.4348 133.8043) (end 38.4348 135.52) (width 0.25) (layer "B.Cu") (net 2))
 (segment (start 38.4348 135.52) (end 41.7654 138.8506) (width 0.25) (layer "B.Cu") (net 2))
 (segment (start 39.2191 133.02) (end 38.4348 133.8043) (width 0.25) (layer "B.Cu") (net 2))
 (segment (start 45.2195 139.8595) (end 61.8042 139.8595) (width 0.25) (layer "B.Cu") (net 13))
 (segment (start 39.65 134.29) (end 45.2195 139.8595) (width 0.25) (layer "B.Cu") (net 13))
 (segment (start 62.4898 139.1739) (end 62.4898 131.6898) (width 0.25) (layer "B.Cu") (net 13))
 (segment (start 62.4898 131.6898) (end 58.77 127.97) (width 0.25) (layer "B.Cu") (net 13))
 (segment (start 61.8042 139.8595) (end 62.4898 139.1739) (width 0.25) (layer "B.Cu") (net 13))
 (segment (start 42.19 134.29) (end 43.46 133.02) (width 0.25) (layer "F.Cu") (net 14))
 (segment (start 43.46 133.02) (end 50.2409 133.02) (width 0.25) (layer "F.Cu") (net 14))
 (segment (start 50.2409 133.02) (end 51.15 132.1109) (width 0.25) (layer "F.Cu") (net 14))
 (segment (start 51.15 132.1109) (end 51.15 127.97) (width 0.25) (layer "F.Cu") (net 14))
 (segment (start 37.11 134.29) (end 38.8602 136.0402) (width 0.25) (layer "F.Cu") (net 12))
 (segment (start 45.5477 136.0402) (end 45.6994 135.8885) (width 0.25) (layer "F.Cu") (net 12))
 (segment (start 51.0978 135.0073) (end 51.0978 133.8245) (width 0.25) (layer "F.Cu") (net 12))
 (segment (start 49.5809 136.5242) (end 51.0978 135.0073) (width 0.25) (layer "F.Cu") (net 12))
 (segment (start 51.0978 133.8245) (end 51.8723 133.05) (width 0.25) (layer "F.Cu") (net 12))
 (segment (start 51.8723 133.05) (end 56.23 133.05) (width 0.25) (layer "F.Cu") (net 12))
 (segment (start 46.937 136.5242) (end 49.5809 136.5242) (width 0.25) (layer "F.Cu") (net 12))
 (segment (start 38.8602 136.0402) (end 45.5477 136.0402) (width 0.25) (layer "F.Cu") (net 12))
 (segment (start 45.6994 135.8885) (end 46.3013 135.8885) (width 0.25) (layer "F.Cu") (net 12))
 (segment (start 56.23 133.05) (end 61.31 127.97) (width 0.25) (layer "F.Cu") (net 12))
 (segment (start 46.3013 135.8885) (end 46.937 136.5242) (width 0.25) (layer "F.Cu") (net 12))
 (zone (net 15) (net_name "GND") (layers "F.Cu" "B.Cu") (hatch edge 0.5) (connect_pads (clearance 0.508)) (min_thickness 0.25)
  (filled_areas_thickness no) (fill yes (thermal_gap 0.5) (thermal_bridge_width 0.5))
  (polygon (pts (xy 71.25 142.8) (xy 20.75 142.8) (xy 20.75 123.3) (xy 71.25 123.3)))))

